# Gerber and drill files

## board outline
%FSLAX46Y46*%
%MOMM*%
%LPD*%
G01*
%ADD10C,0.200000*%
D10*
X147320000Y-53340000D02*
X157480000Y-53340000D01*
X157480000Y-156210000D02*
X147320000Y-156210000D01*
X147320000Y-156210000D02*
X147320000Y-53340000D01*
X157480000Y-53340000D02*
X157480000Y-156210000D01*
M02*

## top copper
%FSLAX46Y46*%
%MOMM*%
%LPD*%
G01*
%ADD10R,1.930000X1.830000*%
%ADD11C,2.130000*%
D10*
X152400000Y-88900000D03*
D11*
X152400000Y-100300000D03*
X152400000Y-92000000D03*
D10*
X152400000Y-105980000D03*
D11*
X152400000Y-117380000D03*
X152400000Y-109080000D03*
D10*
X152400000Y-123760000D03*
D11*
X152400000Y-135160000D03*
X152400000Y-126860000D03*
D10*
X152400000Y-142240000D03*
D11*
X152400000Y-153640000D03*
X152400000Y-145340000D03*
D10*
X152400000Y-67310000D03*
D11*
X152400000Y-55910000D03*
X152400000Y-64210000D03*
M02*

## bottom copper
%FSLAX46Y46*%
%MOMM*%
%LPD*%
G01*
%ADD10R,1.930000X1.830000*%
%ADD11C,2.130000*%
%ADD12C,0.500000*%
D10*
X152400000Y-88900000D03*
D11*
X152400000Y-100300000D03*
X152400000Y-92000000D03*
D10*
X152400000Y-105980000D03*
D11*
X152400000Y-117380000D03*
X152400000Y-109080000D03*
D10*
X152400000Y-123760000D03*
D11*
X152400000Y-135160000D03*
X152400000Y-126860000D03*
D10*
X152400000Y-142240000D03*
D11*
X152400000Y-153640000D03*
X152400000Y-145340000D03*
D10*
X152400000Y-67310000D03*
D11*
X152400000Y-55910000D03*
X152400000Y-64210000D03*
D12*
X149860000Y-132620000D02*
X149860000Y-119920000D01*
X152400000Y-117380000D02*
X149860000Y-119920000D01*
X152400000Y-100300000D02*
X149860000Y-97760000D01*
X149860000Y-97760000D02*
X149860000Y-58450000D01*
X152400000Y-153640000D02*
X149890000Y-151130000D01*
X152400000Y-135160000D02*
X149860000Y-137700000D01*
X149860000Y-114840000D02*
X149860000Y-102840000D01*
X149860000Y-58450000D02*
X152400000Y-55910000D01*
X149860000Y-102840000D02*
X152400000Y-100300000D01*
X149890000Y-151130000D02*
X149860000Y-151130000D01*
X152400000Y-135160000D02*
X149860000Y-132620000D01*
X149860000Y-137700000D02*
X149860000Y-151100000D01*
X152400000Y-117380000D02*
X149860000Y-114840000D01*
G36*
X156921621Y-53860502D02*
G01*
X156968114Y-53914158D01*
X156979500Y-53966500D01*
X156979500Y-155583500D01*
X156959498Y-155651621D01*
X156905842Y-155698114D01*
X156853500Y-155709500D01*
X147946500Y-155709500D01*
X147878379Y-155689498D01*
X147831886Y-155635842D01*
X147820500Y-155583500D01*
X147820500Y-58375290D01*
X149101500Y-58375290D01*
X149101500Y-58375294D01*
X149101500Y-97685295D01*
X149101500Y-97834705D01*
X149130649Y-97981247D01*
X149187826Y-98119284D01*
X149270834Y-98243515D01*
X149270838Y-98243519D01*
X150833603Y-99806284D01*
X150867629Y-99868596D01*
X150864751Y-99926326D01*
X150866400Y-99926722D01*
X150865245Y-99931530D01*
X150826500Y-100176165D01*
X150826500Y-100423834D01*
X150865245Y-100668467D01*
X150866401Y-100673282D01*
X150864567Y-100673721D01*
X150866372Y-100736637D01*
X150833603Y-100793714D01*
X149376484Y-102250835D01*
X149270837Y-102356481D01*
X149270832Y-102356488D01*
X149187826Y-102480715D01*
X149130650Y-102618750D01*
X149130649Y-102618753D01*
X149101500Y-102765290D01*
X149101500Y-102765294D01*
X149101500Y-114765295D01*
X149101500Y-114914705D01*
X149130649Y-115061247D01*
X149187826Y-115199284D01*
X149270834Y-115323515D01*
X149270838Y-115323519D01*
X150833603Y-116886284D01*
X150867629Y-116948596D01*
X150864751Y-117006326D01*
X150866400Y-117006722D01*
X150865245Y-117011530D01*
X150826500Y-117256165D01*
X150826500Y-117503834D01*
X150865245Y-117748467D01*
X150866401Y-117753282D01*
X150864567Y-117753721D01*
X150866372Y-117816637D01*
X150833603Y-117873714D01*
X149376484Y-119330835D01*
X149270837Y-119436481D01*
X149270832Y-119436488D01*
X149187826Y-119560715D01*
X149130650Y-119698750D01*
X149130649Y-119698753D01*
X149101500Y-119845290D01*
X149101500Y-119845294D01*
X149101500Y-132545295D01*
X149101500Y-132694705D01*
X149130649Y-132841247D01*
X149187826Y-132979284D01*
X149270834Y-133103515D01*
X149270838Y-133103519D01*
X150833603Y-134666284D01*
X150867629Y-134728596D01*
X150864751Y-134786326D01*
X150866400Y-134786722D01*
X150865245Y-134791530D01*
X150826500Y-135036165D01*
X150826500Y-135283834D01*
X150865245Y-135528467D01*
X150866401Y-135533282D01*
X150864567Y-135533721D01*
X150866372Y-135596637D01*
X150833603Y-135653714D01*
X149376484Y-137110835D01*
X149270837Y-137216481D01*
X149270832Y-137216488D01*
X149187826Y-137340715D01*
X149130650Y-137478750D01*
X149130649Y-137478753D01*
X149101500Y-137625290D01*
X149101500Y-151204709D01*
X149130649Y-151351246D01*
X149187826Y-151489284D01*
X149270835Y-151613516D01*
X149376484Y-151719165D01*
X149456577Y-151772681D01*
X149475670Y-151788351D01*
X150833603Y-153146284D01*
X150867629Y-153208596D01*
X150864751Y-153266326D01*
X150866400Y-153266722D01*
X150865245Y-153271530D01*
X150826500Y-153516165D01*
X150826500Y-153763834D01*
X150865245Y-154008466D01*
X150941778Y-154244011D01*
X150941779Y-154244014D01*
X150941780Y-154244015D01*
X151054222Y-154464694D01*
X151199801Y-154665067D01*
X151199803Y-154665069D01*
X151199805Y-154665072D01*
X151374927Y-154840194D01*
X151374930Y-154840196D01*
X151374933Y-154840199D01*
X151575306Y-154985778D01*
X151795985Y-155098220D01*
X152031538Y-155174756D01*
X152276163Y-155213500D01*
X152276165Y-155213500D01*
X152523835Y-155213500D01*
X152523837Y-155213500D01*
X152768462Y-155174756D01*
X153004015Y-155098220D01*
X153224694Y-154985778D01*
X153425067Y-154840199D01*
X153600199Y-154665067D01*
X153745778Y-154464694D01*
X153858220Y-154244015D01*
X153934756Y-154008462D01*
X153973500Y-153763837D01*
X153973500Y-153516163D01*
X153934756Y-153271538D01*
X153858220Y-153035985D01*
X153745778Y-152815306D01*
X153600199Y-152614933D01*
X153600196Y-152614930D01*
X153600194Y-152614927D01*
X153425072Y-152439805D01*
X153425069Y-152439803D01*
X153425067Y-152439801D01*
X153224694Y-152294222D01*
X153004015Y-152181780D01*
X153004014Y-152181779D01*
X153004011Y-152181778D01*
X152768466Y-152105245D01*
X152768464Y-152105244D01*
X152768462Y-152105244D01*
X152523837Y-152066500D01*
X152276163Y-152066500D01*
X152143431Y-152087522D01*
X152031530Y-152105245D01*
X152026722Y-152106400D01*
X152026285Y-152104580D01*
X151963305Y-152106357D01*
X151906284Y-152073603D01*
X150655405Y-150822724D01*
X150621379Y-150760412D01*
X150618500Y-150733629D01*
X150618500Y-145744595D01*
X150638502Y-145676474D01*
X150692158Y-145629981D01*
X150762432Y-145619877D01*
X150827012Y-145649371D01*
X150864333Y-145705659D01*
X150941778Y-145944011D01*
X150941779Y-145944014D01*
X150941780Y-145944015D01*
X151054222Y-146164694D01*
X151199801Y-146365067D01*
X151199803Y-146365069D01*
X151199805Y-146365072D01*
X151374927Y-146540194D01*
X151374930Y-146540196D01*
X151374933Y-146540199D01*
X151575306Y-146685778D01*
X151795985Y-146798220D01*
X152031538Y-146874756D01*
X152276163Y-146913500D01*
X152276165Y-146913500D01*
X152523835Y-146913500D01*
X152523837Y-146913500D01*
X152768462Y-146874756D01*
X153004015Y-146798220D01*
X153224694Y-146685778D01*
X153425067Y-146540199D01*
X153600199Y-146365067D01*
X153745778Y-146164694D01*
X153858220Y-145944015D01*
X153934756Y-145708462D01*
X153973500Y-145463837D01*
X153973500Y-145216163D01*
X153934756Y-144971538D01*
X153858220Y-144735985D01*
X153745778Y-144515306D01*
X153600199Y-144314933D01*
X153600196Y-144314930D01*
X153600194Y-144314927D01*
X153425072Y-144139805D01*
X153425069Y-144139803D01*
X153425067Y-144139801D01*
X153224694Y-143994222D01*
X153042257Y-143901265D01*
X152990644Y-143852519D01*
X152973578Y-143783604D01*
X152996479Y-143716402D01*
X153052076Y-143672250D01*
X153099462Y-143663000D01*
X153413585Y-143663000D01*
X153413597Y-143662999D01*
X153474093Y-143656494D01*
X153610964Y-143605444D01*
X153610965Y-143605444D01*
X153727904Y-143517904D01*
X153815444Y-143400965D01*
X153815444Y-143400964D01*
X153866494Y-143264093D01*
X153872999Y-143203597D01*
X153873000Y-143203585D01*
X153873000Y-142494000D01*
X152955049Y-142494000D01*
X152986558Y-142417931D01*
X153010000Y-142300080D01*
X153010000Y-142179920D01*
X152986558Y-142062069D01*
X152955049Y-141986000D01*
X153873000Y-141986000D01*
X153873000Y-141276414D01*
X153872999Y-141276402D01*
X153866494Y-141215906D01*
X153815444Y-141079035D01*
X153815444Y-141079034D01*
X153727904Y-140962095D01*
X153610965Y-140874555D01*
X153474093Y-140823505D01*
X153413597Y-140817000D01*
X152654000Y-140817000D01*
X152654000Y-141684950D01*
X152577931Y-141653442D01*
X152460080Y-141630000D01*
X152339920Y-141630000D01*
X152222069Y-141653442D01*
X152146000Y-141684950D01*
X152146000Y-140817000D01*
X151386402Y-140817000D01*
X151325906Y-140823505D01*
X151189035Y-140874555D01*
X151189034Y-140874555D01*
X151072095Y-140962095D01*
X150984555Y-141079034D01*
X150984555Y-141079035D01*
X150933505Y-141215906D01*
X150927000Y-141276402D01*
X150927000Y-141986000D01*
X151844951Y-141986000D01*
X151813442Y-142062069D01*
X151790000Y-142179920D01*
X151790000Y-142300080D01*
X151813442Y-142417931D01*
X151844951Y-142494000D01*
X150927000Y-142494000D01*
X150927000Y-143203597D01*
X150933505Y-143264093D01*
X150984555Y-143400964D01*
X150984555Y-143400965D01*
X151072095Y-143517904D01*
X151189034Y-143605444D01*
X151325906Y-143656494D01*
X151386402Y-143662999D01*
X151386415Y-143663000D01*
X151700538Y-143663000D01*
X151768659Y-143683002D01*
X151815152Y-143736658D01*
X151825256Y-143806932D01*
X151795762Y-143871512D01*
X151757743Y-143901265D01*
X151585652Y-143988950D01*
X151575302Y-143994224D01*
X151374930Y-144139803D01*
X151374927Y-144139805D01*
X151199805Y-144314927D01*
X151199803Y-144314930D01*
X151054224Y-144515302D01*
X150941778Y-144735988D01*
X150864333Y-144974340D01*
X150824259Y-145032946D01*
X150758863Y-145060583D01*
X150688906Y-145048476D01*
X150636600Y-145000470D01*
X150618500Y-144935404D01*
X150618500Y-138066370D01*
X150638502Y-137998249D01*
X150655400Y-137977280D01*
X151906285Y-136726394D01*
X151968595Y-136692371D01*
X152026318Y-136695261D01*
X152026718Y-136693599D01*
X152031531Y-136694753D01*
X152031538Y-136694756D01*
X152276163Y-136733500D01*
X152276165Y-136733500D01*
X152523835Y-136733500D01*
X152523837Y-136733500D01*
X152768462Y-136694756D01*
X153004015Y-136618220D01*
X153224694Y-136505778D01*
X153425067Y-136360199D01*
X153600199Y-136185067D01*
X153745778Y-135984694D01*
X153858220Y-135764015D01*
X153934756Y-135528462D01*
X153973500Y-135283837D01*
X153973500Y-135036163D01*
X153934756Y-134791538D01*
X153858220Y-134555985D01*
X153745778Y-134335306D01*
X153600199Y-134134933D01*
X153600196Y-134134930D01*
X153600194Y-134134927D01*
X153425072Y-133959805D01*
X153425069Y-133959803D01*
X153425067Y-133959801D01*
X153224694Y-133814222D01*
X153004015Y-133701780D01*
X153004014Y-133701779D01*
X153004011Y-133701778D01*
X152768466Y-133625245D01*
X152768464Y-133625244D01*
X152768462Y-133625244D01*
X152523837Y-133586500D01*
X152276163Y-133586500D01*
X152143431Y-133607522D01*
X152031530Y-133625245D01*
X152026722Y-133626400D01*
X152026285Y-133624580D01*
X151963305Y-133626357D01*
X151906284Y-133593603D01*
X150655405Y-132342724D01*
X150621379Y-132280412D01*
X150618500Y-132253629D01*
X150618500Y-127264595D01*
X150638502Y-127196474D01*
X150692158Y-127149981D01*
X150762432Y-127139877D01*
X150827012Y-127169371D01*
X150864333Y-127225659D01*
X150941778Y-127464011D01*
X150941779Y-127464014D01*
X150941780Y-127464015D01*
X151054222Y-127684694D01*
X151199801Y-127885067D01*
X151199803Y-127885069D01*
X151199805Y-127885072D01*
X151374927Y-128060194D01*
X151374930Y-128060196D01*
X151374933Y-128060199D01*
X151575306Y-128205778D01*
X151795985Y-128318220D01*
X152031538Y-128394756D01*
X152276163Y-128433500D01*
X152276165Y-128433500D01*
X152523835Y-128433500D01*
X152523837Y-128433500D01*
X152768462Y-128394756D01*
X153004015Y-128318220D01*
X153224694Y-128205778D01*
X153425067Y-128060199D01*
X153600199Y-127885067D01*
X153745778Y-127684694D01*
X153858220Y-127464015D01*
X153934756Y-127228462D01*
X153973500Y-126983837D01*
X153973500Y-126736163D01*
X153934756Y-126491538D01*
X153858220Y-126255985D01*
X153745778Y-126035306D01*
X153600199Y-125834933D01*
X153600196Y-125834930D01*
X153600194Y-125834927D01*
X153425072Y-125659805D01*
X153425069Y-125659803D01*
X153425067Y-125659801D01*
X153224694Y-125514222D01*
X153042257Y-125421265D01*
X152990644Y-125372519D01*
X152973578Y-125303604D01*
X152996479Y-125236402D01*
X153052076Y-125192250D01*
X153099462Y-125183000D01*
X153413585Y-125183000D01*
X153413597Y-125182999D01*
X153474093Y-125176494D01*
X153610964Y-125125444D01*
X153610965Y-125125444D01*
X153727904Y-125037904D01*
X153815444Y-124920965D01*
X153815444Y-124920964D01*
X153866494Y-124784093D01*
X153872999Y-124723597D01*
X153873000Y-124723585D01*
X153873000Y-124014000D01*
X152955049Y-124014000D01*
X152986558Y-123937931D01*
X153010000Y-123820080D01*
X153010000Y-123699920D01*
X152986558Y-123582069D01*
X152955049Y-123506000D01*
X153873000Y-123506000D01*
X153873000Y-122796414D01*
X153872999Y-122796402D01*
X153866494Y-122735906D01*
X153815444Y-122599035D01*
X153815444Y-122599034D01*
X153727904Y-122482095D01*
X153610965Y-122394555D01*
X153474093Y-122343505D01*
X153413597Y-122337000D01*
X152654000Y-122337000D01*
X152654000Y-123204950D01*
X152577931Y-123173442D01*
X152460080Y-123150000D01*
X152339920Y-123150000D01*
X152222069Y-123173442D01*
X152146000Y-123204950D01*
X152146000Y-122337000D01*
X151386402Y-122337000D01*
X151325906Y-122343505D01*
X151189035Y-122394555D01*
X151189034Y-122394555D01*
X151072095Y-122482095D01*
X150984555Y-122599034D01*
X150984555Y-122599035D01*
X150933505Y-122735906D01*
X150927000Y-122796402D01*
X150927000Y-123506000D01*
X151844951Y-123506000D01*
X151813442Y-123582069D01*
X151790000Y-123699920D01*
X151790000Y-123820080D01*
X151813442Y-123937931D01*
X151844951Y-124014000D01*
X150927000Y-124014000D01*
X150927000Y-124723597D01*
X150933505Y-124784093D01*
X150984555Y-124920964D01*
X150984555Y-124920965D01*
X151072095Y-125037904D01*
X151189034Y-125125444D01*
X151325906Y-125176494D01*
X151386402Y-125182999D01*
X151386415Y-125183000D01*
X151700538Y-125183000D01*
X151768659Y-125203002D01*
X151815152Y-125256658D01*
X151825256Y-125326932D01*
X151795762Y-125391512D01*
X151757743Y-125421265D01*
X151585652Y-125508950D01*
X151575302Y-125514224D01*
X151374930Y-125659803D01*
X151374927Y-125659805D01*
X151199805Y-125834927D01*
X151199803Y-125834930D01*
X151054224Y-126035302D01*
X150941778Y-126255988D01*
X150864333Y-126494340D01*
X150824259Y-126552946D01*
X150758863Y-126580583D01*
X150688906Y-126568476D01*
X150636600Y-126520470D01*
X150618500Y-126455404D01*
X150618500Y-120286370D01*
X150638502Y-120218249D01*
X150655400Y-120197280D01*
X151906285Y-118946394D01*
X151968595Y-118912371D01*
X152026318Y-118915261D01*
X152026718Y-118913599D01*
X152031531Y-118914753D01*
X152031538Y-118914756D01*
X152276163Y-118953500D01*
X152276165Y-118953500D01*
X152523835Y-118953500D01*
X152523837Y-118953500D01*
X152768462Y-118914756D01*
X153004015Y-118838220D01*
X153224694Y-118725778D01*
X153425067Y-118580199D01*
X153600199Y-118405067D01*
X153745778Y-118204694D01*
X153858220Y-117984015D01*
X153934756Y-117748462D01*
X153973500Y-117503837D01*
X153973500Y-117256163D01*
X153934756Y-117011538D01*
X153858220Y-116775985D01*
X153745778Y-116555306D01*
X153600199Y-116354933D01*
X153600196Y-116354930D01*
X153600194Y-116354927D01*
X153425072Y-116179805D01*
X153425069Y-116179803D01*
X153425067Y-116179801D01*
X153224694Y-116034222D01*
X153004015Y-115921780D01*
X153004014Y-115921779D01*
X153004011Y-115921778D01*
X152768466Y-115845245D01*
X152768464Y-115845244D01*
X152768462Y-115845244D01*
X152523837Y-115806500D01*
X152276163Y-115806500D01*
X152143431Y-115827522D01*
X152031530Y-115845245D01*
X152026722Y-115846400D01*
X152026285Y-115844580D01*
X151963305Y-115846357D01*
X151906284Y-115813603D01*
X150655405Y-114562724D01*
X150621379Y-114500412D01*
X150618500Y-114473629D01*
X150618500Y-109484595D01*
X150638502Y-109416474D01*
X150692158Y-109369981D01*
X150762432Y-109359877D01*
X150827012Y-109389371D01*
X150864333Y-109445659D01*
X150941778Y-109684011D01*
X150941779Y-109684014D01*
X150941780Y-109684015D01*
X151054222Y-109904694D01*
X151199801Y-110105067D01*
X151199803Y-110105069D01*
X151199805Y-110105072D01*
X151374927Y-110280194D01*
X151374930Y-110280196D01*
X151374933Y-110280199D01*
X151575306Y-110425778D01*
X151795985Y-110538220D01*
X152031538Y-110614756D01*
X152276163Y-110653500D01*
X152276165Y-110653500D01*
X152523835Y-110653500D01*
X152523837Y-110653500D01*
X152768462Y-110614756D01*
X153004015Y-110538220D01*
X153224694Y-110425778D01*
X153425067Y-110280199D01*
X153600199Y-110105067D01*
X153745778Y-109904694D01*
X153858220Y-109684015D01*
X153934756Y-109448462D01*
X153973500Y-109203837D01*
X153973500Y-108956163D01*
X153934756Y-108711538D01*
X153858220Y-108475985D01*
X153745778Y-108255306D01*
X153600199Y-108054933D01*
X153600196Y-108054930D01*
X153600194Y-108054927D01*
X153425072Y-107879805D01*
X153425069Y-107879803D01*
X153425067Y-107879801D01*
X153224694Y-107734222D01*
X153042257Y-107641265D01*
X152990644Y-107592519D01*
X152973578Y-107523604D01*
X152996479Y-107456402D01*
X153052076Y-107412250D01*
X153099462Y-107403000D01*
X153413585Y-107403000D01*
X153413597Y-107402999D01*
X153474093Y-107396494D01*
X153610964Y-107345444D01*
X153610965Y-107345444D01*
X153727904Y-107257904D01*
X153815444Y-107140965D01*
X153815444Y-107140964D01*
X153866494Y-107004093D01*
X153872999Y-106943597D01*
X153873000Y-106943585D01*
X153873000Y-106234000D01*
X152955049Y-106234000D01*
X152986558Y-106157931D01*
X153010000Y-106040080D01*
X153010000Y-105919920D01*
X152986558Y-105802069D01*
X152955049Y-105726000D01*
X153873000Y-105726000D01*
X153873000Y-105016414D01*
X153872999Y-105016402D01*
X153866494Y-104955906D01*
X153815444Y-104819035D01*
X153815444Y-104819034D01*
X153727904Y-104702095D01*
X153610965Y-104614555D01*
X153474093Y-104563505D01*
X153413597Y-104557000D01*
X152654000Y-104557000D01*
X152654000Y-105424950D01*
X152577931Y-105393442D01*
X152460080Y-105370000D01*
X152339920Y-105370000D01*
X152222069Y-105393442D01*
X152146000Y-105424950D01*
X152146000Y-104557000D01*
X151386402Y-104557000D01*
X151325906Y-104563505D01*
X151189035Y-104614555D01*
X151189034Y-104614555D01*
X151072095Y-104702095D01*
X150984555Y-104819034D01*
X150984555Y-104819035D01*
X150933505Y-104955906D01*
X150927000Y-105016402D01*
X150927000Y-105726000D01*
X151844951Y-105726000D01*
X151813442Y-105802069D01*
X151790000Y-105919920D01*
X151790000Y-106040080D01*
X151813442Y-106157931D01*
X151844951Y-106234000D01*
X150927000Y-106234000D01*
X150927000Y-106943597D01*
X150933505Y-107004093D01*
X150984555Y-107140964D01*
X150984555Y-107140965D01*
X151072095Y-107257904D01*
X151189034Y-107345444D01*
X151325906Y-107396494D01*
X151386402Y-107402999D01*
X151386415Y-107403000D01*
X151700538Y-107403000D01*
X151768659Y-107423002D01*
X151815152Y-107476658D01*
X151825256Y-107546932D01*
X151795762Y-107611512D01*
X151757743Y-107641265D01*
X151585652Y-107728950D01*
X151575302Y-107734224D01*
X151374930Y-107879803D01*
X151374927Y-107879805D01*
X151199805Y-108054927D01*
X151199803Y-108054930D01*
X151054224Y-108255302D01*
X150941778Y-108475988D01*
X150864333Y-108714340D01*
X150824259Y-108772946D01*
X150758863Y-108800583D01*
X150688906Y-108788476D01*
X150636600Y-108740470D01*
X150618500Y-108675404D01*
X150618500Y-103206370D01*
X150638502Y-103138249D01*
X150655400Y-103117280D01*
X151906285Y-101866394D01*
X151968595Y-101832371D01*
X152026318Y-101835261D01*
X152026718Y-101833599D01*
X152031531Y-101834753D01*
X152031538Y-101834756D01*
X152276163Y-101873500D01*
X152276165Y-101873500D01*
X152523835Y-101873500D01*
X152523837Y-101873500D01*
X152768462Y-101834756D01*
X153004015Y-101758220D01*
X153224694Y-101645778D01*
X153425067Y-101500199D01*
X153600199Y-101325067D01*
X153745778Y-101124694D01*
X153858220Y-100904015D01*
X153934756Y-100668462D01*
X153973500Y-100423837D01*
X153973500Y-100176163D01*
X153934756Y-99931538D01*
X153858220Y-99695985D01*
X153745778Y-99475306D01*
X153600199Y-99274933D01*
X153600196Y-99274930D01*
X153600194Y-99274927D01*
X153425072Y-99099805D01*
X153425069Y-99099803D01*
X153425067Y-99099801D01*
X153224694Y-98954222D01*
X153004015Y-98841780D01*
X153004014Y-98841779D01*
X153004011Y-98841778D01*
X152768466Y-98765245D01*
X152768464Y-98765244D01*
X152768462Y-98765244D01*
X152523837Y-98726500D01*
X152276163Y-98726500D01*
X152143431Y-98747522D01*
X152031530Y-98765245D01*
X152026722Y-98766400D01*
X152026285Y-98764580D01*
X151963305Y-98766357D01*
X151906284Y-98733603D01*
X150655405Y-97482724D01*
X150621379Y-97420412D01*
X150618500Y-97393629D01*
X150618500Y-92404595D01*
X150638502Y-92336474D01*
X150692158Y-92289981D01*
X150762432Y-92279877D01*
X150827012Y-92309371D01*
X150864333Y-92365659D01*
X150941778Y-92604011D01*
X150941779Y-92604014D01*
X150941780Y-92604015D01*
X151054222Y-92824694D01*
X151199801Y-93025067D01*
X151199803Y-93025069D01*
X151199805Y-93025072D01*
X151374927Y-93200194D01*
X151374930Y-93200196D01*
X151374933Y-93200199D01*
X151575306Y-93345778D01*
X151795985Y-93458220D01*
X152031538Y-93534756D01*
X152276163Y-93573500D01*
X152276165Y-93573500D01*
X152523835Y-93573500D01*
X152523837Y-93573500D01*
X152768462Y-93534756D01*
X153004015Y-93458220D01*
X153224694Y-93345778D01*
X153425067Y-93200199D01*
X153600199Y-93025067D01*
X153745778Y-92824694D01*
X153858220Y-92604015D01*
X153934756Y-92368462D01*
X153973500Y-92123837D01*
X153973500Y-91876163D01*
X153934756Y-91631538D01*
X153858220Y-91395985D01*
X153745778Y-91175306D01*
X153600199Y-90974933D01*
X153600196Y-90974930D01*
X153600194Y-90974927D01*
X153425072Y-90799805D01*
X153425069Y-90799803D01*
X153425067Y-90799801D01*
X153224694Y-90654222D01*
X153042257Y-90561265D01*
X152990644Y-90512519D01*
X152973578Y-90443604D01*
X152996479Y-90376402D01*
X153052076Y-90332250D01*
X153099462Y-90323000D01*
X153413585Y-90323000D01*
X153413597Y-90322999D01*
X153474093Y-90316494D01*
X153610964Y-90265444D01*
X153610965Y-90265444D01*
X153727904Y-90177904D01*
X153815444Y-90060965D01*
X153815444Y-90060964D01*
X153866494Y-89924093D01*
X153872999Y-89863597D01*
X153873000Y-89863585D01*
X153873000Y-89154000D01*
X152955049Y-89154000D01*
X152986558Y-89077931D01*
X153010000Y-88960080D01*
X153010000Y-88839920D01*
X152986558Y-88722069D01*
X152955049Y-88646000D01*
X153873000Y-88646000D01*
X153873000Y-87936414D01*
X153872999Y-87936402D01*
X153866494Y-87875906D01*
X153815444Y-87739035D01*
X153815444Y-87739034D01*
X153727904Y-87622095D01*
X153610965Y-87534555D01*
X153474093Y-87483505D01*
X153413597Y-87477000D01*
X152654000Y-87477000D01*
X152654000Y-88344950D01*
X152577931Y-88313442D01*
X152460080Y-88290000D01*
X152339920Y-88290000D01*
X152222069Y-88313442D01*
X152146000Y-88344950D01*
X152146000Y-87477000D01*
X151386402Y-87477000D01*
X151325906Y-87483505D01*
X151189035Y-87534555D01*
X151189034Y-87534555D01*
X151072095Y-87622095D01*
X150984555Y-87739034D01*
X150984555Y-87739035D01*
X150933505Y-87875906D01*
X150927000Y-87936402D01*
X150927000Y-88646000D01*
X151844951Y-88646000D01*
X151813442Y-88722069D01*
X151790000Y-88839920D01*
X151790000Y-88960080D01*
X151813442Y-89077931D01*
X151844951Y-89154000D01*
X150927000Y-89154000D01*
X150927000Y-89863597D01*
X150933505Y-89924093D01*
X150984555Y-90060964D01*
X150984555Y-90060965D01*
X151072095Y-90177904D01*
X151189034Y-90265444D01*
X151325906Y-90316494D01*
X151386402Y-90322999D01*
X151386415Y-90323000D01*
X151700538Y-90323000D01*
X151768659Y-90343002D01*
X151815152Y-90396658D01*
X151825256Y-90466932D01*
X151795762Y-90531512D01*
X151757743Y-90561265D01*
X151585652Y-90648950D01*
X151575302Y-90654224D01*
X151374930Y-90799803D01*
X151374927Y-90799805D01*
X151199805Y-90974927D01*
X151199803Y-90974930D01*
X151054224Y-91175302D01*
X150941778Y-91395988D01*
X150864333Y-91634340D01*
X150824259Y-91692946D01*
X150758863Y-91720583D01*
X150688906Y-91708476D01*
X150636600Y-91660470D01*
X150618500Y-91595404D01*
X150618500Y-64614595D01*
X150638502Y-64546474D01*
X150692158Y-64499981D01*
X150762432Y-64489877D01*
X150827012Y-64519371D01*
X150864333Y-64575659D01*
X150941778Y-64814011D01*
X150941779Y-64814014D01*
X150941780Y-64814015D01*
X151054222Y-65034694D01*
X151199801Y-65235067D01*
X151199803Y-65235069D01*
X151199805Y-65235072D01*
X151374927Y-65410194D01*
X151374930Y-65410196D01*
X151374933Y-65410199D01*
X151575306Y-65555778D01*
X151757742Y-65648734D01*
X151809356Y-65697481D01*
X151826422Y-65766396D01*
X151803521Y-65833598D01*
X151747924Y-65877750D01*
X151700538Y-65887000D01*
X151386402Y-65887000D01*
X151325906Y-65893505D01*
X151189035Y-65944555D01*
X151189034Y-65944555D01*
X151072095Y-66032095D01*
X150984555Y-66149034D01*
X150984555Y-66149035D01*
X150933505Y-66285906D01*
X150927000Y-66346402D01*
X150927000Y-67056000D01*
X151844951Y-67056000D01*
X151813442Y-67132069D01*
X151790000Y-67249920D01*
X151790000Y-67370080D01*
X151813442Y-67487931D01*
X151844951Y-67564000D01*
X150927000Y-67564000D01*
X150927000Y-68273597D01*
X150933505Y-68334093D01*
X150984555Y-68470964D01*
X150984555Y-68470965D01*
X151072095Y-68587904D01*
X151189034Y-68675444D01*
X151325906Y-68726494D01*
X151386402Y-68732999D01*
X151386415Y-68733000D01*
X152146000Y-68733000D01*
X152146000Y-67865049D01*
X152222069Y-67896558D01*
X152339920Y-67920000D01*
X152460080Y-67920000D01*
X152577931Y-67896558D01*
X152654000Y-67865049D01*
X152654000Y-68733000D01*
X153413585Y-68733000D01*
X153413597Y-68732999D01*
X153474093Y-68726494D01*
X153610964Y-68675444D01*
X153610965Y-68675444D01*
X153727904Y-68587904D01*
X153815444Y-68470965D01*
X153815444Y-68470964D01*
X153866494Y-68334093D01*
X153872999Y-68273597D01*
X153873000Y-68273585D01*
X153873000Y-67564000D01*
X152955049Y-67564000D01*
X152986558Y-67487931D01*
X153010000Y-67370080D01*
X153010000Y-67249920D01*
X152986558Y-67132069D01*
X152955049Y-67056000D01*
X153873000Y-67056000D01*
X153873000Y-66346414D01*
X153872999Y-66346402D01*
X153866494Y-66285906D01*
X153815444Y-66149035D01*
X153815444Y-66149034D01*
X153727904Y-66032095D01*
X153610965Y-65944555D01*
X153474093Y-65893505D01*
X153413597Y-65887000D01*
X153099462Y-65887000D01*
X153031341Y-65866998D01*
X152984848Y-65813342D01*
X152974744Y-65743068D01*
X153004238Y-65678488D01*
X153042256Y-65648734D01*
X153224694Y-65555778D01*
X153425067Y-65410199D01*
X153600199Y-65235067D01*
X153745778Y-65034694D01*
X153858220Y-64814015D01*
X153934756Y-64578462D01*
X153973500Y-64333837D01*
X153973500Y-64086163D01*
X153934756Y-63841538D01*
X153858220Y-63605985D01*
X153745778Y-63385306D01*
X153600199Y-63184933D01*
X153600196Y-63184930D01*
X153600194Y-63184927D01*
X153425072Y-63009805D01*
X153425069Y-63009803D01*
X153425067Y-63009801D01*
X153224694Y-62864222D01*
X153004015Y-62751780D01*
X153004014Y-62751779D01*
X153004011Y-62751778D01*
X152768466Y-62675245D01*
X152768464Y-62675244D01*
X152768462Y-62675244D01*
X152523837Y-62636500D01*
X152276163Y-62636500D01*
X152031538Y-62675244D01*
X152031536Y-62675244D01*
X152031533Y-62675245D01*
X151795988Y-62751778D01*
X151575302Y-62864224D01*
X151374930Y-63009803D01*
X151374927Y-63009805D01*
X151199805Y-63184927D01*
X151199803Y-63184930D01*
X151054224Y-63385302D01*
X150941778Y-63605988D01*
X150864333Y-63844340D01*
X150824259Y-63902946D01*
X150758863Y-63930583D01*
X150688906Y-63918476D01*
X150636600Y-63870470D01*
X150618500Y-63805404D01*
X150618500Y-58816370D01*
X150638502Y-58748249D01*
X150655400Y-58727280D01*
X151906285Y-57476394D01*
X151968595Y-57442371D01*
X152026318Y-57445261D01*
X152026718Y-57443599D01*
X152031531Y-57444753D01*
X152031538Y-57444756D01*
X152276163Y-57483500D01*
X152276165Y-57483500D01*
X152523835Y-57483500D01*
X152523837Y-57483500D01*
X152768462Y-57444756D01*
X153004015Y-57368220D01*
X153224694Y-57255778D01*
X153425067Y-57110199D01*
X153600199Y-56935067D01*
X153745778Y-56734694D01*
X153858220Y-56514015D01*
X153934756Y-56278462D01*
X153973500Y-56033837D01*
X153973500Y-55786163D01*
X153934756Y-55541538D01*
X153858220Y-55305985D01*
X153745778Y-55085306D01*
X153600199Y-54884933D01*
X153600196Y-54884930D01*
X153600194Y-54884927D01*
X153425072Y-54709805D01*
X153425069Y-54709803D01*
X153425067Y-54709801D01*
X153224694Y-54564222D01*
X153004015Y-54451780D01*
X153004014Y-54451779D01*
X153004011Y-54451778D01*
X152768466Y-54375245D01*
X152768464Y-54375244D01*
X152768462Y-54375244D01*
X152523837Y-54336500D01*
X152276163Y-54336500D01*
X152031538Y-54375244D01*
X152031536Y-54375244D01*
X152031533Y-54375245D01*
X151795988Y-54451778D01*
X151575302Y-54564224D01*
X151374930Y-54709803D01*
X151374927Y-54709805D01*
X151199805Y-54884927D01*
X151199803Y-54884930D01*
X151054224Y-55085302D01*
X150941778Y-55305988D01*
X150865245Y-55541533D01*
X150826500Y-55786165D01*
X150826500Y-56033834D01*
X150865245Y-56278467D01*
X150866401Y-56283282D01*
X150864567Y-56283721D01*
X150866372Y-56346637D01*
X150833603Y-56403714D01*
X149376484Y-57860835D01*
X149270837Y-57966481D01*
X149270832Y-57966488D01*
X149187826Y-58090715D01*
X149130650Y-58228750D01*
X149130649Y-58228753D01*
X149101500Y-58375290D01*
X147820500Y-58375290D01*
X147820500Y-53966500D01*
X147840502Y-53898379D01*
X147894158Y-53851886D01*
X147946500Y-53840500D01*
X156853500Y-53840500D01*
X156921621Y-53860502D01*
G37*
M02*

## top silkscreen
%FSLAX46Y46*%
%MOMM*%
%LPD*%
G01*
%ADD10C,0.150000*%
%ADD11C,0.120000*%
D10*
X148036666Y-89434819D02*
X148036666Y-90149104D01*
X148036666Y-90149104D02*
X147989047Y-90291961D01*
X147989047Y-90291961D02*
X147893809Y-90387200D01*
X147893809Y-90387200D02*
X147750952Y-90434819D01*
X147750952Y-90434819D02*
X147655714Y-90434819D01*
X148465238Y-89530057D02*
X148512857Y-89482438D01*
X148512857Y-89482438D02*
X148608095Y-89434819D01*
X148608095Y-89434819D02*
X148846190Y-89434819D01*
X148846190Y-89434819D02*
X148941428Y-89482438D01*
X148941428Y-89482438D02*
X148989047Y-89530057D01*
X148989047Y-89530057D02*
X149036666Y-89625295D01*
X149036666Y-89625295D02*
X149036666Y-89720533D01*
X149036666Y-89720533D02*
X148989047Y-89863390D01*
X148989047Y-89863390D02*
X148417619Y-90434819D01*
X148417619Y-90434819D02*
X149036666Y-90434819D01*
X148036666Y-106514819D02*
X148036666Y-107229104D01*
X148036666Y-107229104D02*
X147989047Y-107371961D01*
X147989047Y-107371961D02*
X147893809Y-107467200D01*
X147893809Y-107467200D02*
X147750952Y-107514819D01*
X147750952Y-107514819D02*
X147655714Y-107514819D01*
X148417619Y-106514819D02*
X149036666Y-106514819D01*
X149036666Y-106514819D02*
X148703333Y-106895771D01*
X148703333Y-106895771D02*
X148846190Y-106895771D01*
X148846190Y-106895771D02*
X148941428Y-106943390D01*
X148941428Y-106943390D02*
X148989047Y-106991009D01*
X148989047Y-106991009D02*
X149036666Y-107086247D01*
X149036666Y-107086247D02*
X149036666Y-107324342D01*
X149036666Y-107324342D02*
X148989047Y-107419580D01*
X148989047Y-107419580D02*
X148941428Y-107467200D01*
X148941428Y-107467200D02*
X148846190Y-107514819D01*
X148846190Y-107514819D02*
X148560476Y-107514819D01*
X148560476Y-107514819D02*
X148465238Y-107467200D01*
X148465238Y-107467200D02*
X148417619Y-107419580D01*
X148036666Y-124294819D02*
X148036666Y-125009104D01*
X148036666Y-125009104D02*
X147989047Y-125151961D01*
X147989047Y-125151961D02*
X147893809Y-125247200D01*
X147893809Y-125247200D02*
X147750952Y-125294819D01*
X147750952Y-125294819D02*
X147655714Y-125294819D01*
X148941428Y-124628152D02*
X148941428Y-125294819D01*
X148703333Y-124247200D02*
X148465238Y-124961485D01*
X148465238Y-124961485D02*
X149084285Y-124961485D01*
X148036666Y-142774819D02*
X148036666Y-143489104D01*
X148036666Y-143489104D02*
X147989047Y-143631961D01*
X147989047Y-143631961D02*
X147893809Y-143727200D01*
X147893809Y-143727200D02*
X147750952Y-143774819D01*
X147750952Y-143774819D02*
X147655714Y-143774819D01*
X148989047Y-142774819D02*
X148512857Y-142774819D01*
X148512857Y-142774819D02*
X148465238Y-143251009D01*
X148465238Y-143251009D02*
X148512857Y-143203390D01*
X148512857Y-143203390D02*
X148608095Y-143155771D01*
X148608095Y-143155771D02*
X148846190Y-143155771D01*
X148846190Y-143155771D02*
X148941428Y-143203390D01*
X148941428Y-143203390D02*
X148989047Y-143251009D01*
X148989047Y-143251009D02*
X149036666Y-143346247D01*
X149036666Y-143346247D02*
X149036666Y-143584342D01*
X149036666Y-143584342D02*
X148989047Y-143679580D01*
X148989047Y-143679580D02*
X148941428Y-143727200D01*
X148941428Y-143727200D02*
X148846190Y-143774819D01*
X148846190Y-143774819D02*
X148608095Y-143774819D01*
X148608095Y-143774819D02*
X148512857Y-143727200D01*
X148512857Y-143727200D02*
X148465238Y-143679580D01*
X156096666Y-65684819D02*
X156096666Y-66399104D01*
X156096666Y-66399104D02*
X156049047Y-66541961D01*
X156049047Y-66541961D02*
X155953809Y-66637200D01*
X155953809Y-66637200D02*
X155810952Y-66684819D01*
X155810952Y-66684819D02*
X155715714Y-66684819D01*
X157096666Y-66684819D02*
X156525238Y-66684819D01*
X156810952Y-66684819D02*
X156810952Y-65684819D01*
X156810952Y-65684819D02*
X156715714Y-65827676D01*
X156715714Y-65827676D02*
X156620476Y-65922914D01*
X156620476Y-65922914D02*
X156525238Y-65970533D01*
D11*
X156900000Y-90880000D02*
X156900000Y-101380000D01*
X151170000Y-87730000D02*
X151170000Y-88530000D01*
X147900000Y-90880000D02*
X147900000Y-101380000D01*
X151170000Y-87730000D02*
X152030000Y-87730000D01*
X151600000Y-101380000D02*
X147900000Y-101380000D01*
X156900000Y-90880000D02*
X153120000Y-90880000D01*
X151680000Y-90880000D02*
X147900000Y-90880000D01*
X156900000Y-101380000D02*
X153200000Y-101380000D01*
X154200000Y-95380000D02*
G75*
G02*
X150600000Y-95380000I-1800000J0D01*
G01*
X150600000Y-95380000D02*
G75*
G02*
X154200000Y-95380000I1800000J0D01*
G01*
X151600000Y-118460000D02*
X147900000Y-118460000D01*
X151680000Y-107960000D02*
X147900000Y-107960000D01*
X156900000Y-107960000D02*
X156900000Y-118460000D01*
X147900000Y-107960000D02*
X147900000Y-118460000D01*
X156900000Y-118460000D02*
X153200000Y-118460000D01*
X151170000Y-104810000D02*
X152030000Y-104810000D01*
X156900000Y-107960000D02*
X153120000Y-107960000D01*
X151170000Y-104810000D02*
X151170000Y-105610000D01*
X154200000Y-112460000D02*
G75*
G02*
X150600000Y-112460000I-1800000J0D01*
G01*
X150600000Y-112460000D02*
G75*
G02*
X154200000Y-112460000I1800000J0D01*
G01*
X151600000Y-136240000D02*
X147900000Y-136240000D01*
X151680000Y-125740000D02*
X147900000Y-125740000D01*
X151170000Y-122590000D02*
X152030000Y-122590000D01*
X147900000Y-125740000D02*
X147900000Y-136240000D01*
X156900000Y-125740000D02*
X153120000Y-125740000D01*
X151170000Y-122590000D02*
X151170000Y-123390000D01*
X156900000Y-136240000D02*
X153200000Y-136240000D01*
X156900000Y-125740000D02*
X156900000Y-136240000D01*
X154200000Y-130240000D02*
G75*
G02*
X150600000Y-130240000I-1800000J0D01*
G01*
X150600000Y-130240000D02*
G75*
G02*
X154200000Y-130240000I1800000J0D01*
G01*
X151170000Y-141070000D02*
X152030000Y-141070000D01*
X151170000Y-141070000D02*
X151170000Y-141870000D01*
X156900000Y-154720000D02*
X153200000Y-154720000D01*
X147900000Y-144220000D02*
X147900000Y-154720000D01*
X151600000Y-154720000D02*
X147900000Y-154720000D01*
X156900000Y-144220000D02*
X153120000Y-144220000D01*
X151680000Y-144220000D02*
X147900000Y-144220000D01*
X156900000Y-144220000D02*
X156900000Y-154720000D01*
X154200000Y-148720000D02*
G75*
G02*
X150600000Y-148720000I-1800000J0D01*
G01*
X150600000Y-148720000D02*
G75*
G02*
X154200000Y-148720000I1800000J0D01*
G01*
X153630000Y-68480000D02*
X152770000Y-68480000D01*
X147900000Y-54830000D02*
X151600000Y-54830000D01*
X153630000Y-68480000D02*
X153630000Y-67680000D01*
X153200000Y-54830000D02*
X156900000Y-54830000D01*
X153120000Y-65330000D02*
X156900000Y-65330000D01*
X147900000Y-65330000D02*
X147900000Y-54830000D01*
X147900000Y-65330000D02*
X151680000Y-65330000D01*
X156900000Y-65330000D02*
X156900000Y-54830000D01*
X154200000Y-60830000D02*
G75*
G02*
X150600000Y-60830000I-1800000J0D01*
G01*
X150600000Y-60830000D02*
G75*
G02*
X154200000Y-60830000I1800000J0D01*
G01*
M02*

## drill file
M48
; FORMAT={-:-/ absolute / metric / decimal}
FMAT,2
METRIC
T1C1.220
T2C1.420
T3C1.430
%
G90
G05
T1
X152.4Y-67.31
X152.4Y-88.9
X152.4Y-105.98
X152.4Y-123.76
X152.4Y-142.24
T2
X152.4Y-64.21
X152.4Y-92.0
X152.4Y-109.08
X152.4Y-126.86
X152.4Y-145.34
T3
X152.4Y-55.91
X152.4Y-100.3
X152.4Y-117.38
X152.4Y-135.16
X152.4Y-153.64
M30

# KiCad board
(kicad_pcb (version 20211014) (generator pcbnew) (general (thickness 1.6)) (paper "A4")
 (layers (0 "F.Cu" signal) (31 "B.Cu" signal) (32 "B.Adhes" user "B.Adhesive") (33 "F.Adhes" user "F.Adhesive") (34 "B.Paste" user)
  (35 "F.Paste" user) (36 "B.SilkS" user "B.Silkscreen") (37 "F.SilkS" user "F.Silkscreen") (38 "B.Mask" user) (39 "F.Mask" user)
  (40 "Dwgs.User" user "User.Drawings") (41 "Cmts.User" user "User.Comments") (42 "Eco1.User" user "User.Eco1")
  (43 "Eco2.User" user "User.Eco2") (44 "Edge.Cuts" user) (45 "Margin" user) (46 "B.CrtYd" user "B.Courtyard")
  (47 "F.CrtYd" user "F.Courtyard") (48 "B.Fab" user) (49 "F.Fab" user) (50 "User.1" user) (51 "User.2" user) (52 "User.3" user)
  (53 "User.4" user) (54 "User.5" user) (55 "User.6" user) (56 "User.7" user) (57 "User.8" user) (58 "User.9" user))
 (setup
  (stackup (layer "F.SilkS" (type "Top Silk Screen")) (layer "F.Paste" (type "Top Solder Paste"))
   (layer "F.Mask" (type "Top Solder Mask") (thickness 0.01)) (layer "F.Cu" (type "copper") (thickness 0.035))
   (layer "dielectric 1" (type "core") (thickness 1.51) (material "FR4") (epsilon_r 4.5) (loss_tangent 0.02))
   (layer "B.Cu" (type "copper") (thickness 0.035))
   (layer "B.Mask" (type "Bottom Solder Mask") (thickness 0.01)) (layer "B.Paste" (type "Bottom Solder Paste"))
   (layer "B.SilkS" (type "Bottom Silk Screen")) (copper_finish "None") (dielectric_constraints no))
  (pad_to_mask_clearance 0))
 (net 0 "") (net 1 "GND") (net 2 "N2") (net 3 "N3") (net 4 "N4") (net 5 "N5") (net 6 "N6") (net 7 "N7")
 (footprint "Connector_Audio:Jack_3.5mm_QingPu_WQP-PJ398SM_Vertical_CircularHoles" (layer "F.Cu") (at 152.4 88.9)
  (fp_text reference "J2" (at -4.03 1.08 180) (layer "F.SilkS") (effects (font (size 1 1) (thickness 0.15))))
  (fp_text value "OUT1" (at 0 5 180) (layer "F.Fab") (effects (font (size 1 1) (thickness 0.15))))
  (fp_line (start 4.5 1.98) (end 4.5 12.48) (layer "F.SilkS") (width 0.12))
  (fp_line (start -1.23 -1.17) (end -1.23 -0.37) (layer "F.SilkS") (width 0.12))
  (fp_line (start -4.5 1.98) (end -4.5 12.48) (layer "F.SilkS") (width 0.12))
  (fp_line (start -1.23 -1.17) (end -0.37 -1.17) (layer "F.SilkS") (width 0.12))
  (fp_line (start -0.8 12.48) (end -4.5 12.48) (layer "F.SilkS") (width 0.12))
  (fp_line (start 4.5 1.98) (end 0.72 1.98) (layer "F.SilkS") (width 0.12))
  (fp_line (start -0.72 1.98) (end -4.5 1.98) (layer "F.SilkS") (width 0.12))
  (fp_line (start 4.5 12.48) (end 0.8 12.48) (layer "F.SilkS") (width 0.12))
  (fp_circle (center 0 6.48) (end 1.8 6.48) (layer "F.SilkS") (width 0.12) (fill none))
  (pad "S" thru_hole rect (at 0 0 180) (size 1.93 1.83) (drill 1.22) (layers *.Cu *.Mask) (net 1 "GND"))
  (pad "T" thru_hole circle (at 0 11.4 180) (size 2.13 2.13) (drill 1.43) (layers *.Cu *.Mask) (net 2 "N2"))
  (pad "TN" thru_hole circle (at 0 3.1 180) (size 2.13 2.13) (drill 1.42) (layers *.Cu *.Mask) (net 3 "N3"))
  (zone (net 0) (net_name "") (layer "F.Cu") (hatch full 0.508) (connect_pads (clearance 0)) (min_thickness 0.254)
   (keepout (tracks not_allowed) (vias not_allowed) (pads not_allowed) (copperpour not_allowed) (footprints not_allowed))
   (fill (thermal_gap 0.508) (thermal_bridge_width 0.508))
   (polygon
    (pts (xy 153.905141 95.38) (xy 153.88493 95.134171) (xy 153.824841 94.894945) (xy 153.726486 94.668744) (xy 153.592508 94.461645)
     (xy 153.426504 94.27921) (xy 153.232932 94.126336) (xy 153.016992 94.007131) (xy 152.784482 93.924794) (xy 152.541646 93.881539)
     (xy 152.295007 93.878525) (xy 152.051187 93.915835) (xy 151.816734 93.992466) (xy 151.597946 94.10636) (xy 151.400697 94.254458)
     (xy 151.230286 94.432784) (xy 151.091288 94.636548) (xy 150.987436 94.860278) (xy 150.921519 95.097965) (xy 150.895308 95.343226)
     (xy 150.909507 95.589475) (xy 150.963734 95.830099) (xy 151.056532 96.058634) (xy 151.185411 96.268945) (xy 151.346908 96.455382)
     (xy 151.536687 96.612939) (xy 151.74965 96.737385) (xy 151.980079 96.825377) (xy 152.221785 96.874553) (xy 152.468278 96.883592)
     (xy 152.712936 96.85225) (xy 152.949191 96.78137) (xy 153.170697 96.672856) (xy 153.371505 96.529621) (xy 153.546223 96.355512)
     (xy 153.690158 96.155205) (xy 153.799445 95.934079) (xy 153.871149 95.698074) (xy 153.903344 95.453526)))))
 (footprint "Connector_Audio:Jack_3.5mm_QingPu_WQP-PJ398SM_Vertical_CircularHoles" (layer "F.Cu") (at 152.4 105.98)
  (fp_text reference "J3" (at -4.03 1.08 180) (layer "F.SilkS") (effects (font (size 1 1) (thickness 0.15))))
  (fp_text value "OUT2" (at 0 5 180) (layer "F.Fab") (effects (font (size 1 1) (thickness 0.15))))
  (fp_line (start -0.8 12.48) (end -4.5 12.48) (layer "F.SilkS") (width 0.12))
  (fp_line (start -0.72 1.98) (end -4.5 1.98) (layer "F.SilkS") (width 0.12))
  (fp_line (start 4.5 1.98) (end 4.5 12.48) (layer "F.SilkS") (width 0.12))
  (fp_line (start -4.5 1.98) (end -4.5 12.48) (layer "F.SilkS") (width 0.12))
  (fp_line (start 4.5 12.48) (end 0.8 12.48) (layer "F.SilkS") (width 0.12))
  (fp_line (start -1.23 -1.17) (end -0.37 -1.17) (layer "F.SilkS") (width 0.12))
  (fp_line (start 4.5 1.98) (end 0.72 1.98) (layer "F.SilkS") (width 0.12))
  (fp_line (start -1.23 -1.17) (end -1.23 -0.37) (layer "F.SilkS") (width 0.12))
  (fp_circle (center 0 6.48) (end 1.8 6.48) (layer "F.SilkS") (width 0.12) (fill none))
  (pad "S" thru_hole rect (at 0 0 180) (size 1.93 1.83) (drill 1.22) (layers *.Cu *.Mask) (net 1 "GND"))
  (pad "T" thru_hole circle (at 0 11.4 180) (size 2.13 2.13) (drill 1.43) (layers *.Cu *.Mask) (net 2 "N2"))
  (pad "TN" thru_hole circle (at 0 3.1 180) (size 2.13 2.13) (drill 1.42) (layers *.Cu *.Mask) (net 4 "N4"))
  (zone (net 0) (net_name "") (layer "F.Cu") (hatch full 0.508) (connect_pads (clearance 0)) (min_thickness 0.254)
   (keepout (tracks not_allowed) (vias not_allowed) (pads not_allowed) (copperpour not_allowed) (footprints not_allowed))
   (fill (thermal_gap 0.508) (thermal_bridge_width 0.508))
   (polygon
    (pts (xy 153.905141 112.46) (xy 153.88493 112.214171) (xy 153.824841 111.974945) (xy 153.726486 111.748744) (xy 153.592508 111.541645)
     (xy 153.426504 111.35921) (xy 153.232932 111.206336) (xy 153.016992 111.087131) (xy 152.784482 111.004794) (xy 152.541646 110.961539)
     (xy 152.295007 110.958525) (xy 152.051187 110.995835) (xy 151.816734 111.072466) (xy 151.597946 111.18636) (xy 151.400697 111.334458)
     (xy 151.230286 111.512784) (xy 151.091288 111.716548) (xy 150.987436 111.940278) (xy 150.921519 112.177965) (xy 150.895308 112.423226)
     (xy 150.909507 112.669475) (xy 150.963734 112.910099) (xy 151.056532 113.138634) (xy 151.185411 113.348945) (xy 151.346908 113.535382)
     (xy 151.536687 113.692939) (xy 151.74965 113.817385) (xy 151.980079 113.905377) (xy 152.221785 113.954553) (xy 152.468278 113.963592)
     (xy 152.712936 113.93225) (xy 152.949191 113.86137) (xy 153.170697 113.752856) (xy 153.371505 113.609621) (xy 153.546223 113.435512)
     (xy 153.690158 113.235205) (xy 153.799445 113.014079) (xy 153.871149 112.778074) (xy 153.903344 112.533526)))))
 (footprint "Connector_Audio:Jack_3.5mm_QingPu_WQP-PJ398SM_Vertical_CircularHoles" (layer "F.Cu") (at 152.4 123.76)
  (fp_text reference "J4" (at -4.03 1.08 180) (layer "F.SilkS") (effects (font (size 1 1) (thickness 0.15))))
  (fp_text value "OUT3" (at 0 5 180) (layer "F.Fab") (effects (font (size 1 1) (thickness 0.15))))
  (fp_line (start -0.8 12.48) (end -4.5 12.48) (layer "F.SilkS") (width 0.12))
  (fp_line (start -0.72 1.98) (end -4.5 1.98) (layer "F.SilkS") (width 0.12))
  (fp_line (start -1.23 -1.17) (end -0.37 -1.17) (layer "F.SilkS") (width 0.12))
  (fp_line (start -4.5 1.98) (end -4.5 12.48) (layer "F.SilkS") (width 0.12))
  (fp_line (start 4.5 1.98) (end 0.72 1.98) (layer "F.SilkS") (width 0.12))
  (fp_line (start -1.23 -1.17) (end -1.23 -0.37) (layer "F.SilkS") (width 0.12))
  (fp_line (start 4.5 12.48) (end 0.8 12.48) (layer "F.SilkS") (width 0.12))
  (fp_line (start 4.5 1.98) (end 4.5 12.48) (layer "F.SilkS") (width 0.12))
  (fp_circle (center 0 6.48) (end 1.8 6.48) (layer "F.SilkS") (width 0.12) (fill none))
  (pad "S" thru_hole rect (at 0 0 180) (size 1.93 1.83) (drill 1.22) (layers *.Cu *.Mask) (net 1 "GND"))
  (pad "T" thru_hole circle (at 0 11.4 180) (size 2.13 2.13) (drill 1.43) (layers *.Cu *.Mask) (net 2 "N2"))
  (pad "TN" thru_hole circle (at 0 3.1 180) (size 2.13 2.13) (drill 1.42) (layers *.Cu *.Mask) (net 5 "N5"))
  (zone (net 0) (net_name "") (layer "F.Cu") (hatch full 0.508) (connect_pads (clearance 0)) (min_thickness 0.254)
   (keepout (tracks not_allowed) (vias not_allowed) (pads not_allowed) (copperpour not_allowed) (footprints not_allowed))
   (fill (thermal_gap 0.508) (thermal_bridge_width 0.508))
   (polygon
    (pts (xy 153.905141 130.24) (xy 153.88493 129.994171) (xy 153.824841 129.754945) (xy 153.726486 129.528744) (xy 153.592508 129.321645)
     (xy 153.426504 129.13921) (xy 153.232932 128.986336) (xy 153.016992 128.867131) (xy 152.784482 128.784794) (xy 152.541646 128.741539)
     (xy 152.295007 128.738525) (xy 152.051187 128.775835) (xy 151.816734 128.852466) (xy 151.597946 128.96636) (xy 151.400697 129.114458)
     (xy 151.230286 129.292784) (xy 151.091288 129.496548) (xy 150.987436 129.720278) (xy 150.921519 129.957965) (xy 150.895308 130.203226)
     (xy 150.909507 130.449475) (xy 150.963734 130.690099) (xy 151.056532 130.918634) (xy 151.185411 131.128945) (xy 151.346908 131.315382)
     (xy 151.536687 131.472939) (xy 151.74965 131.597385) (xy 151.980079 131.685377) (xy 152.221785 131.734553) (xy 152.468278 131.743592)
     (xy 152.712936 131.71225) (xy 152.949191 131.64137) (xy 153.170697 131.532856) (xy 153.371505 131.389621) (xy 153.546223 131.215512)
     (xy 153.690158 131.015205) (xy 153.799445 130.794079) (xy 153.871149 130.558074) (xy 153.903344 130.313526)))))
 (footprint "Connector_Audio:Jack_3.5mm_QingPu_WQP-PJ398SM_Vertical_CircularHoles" (layer "F.Cu") (at 152.4 142.24)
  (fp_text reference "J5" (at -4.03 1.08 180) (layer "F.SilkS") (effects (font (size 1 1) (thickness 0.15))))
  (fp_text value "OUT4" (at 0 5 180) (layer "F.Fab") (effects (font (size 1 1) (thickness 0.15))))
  (fp_line (start -1.23 -1.17) (end -0.37 -1.17) (layer "F.SilkS") (width 0.12))
  (fp_line (start -1.23 -1.17) (end -1.23 -0.37) (layer "F.SilkS") (width 0.12))
  (fp_line (start 4.5 12.48) (end 0.8 12.48) (layer "F.SilkS") (width 0.12))
  (fp_line (start -4.5 1.98) (end -4.5 12.48) (layer "F.SilkS") (width 0.12))
  (fp_line (start -0.8 12.48) (end -4.5 12.48) (layer "F.SilkS") (width 0.12))
  (fp_line (start 4.5 1.98) (end 0.72 1.98) (layer "F.SilkS") (width 0.12))
  (fp_line (start -0.72 1.98) (end -4.5 1.98) (layer "F.SilkS") (width 0.12))
  (fp_line (start 4.5 1.98) (end 4.5 12.48) (layer "F.SilkS") (width 0.12))
  (fp_circle (center 0 6.48) (end 1.8 6.48) (layer "F.SilkS") (width 0.12) (fill none))
  (pad "S" thru_hole rect (at 0 0 180) (size 1.93 1.83) (drill 1.22) (layers *.Cu *.Mask) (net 1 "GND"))
  (pad "T" thru_hole circle (at 0 11.4 180) (size 2.13 2.13) (drill 1.43) (layers *.Cu *.Mask) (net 2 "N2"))
  (pad "TN" thru_hole circle (at 0 3.1 180) (size 2.13 2.13) (drill 1.42) (layers *.Cu *.Mask) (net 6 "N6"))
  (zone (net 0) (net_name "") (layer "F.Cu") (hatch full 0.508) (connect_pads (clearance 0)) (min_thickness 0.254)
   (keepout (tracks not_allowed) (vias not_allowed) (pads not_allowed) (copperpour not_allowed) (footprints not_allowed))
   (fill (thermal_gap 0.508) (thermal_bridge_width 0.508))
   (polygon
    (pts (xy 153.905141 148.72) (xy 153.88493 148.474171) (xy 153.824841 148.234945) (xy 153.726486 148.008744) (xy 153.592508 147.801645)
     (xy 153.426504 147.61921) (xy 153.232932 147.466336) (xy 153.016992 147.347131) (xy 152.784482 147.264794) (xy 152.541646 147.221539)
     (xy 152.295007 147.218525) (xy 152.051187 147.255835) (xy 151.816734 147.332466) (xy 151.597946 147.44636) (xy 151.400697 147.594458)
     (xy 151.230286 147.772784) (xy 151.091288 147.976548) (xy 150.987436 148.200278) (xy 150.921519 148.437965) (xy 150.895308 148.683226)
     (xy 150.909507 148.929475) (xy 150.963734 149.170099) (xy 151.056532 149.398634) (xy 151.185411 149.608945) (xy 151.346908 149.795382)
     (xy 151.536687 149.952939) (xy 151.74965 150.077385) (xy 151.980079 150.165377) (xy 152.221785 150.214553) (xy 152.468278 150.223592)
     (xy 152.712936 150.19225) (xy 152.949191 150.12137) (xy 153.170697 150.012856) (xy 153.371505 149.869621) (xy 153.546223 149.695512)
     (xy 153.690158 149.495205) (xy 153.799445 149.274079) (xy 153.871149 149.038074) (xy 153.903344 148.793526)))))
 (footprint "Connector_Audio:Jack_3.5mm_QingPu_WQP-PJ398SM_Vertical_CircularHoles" (layer "F.Cu") (at 152.4 67.31 180)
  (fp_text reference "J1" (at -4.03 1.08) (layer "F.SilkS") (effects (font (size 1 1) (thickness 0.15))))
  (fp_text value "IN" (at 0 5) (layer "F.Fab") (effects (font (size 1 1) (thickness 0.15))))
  (fp_line (start -1.23 -1.17) (end -0.37 -1.17) (layer "F.SilkS") (width 0.12))
  (fp_line (start 4.5 12.48) (end 0.8 12.48) (layer "F.SilkS") (width 0.12))
  (fp_line (start -1.23 -1.17) (end -1.23 -0.37) (layer "F.SilkS") (width 0.12))
  (fp_line (start -0.8 12.48) (end -4.5 12.48) (layer "F.SilkS") (width 0.12))
  (fp_line (start -0.72 1.98) (end -4.5 1.98) (layer "F.SilkS") (width 0.12))
  (fp_line (start 4.5 1.98) (end 4.5 12.48) (layer "F.SilkS") (width 0.12))
  (fp_line (start 4.5 1.98) (end 0.72 1.98) (layer "F.SilkS") (width 0.12))
  (fp_line (start -4.5 1.98) (end -4.5 12.48) (layer "F.SilkS") (width 0.12))
  (fp_circle (center 0 6.48) (end 1.8 6.48) (layer "F.SilkS") (width 0.12) (fill none))
  (pad "S" thru_hole rect (at 0 0) (size 1.93 1.83) (drill 1.22) (layers *.Cu *.Mask) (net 1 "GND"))
  (pad "T" thru_hole circle (at 0 11.4) (size 2.13 2.13) (drill 1.43) (layers *.Cu *.Mask) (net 2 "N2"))
  (pad "TN" thru_hole circle (at 0 3.1) (size 2.13 2.13) (drill 1.42) (layers *.Cu *.Mask) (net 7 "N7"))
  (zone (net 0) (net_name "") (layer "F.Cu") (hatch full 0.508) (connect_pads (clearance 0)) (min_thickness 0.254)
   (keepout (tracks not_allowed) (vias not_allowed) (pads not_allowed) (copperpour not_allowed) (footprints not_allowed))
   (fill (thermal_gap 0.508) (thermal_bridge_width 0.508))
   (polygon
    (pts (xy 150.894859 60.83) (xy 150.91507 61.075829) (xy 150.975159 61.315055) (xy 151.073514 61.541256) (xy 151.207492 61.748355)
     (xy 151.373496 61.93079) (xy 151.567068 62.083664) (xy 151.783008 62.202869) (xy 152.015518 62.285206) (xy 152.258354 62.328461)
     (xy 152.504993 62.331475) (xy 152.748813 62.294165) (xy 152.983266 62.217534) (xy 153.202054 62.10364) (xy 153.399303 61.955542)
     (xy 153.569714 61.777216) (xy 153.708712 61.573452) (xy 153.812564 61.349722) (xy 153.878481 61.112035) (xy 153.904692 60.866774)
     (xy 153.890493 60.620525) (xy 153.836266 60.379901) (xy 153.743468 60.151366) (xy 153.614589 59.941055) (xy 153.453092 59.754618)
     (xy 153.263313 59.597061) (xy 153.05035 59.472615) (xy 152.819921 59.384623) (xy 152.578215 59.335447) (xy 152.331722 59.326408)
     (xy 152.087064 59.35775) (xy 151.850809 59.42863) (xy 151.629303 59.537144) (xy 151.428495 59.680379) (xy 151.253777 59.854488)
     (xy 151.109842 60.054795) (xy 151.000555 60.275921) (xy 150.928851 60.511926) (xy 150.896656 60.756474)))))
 (gr_line (start 147.32 53.34) (end 157.48 53.34) (layer "Edge.Cuts") (width 0.2))
 (gr_line (start 157.48 156.21) (end 147.32 156.21) (layer "Edge.Cuts") (width 0.2))
 (gr_line (start 147.32 156.21) (end 147.32 53.34) (layer "Edge.Cuts") (width 0.2))
 (gr_line (start 157.48 53.34) (end 157.48 156.21) (layer "Edge.Cuts") (width 0.2))
 (segment (start 149.86 132.62) (end 149.86 119.92) (width 0.5) (layer "B.Cu") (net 2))
 (segment (start 152.4 117.38) (end 149.86 119.92) (width 0.5) (layer "B.Cu") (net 2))
 (segment (start 152.4 100.3) (end 149.86 97.76) (width 0.5) (layer "B.Cu") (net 2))
 (segment (start 149.86 97.76) (end 149.86 58.45) (width 0.5) (layer "B.Cu") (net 2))
 (segment (start 152.4 153.64) (end 149.89 151.13) (width 0.5) (layer "B.Cu") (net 2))
 (segment (start 152.4 135.16) (end 149.86 137.7) (width 0.5) (layer "B.Cu") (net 2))
 (segment (start 149.86 114.84) (end 149.86 102.84) (width 0.5) (layer "B.Cu") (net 2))
 (segment (start 149.86 58.45) (end 152.4 55.91) (width 0.5) (layer "B.Cu") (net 2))
 (segment (start 149.86 102.84) (end 152.4 100.3) (width 0.5) (layer "B.Cu") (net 2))
 (segment (start 149.89 151.13) (end 149.86 151.13) (width 0.5) (layer "B.Cu") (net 2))
 (segment (start 152.4 135.16) (end 149.86 132.62) (width 0.5) (layer "B.Cu") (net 2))
 (segment (start 149.86 137.7) (end 149.86 151.1) (width 0.5) (layer "B.Cu") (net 2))
 (segment (start 152.4 117.38) (end 149.86 114.84) (width 0.5) (layer "B.Cu") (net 2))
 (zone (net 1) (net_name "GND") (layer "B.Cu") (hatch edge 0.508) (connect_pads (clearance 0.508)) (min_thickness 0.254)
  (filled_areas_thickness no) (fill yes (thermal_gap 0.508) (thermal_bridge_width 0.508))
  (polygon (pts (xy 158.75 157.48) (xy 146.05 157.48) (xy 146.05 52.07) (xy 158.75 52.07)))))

